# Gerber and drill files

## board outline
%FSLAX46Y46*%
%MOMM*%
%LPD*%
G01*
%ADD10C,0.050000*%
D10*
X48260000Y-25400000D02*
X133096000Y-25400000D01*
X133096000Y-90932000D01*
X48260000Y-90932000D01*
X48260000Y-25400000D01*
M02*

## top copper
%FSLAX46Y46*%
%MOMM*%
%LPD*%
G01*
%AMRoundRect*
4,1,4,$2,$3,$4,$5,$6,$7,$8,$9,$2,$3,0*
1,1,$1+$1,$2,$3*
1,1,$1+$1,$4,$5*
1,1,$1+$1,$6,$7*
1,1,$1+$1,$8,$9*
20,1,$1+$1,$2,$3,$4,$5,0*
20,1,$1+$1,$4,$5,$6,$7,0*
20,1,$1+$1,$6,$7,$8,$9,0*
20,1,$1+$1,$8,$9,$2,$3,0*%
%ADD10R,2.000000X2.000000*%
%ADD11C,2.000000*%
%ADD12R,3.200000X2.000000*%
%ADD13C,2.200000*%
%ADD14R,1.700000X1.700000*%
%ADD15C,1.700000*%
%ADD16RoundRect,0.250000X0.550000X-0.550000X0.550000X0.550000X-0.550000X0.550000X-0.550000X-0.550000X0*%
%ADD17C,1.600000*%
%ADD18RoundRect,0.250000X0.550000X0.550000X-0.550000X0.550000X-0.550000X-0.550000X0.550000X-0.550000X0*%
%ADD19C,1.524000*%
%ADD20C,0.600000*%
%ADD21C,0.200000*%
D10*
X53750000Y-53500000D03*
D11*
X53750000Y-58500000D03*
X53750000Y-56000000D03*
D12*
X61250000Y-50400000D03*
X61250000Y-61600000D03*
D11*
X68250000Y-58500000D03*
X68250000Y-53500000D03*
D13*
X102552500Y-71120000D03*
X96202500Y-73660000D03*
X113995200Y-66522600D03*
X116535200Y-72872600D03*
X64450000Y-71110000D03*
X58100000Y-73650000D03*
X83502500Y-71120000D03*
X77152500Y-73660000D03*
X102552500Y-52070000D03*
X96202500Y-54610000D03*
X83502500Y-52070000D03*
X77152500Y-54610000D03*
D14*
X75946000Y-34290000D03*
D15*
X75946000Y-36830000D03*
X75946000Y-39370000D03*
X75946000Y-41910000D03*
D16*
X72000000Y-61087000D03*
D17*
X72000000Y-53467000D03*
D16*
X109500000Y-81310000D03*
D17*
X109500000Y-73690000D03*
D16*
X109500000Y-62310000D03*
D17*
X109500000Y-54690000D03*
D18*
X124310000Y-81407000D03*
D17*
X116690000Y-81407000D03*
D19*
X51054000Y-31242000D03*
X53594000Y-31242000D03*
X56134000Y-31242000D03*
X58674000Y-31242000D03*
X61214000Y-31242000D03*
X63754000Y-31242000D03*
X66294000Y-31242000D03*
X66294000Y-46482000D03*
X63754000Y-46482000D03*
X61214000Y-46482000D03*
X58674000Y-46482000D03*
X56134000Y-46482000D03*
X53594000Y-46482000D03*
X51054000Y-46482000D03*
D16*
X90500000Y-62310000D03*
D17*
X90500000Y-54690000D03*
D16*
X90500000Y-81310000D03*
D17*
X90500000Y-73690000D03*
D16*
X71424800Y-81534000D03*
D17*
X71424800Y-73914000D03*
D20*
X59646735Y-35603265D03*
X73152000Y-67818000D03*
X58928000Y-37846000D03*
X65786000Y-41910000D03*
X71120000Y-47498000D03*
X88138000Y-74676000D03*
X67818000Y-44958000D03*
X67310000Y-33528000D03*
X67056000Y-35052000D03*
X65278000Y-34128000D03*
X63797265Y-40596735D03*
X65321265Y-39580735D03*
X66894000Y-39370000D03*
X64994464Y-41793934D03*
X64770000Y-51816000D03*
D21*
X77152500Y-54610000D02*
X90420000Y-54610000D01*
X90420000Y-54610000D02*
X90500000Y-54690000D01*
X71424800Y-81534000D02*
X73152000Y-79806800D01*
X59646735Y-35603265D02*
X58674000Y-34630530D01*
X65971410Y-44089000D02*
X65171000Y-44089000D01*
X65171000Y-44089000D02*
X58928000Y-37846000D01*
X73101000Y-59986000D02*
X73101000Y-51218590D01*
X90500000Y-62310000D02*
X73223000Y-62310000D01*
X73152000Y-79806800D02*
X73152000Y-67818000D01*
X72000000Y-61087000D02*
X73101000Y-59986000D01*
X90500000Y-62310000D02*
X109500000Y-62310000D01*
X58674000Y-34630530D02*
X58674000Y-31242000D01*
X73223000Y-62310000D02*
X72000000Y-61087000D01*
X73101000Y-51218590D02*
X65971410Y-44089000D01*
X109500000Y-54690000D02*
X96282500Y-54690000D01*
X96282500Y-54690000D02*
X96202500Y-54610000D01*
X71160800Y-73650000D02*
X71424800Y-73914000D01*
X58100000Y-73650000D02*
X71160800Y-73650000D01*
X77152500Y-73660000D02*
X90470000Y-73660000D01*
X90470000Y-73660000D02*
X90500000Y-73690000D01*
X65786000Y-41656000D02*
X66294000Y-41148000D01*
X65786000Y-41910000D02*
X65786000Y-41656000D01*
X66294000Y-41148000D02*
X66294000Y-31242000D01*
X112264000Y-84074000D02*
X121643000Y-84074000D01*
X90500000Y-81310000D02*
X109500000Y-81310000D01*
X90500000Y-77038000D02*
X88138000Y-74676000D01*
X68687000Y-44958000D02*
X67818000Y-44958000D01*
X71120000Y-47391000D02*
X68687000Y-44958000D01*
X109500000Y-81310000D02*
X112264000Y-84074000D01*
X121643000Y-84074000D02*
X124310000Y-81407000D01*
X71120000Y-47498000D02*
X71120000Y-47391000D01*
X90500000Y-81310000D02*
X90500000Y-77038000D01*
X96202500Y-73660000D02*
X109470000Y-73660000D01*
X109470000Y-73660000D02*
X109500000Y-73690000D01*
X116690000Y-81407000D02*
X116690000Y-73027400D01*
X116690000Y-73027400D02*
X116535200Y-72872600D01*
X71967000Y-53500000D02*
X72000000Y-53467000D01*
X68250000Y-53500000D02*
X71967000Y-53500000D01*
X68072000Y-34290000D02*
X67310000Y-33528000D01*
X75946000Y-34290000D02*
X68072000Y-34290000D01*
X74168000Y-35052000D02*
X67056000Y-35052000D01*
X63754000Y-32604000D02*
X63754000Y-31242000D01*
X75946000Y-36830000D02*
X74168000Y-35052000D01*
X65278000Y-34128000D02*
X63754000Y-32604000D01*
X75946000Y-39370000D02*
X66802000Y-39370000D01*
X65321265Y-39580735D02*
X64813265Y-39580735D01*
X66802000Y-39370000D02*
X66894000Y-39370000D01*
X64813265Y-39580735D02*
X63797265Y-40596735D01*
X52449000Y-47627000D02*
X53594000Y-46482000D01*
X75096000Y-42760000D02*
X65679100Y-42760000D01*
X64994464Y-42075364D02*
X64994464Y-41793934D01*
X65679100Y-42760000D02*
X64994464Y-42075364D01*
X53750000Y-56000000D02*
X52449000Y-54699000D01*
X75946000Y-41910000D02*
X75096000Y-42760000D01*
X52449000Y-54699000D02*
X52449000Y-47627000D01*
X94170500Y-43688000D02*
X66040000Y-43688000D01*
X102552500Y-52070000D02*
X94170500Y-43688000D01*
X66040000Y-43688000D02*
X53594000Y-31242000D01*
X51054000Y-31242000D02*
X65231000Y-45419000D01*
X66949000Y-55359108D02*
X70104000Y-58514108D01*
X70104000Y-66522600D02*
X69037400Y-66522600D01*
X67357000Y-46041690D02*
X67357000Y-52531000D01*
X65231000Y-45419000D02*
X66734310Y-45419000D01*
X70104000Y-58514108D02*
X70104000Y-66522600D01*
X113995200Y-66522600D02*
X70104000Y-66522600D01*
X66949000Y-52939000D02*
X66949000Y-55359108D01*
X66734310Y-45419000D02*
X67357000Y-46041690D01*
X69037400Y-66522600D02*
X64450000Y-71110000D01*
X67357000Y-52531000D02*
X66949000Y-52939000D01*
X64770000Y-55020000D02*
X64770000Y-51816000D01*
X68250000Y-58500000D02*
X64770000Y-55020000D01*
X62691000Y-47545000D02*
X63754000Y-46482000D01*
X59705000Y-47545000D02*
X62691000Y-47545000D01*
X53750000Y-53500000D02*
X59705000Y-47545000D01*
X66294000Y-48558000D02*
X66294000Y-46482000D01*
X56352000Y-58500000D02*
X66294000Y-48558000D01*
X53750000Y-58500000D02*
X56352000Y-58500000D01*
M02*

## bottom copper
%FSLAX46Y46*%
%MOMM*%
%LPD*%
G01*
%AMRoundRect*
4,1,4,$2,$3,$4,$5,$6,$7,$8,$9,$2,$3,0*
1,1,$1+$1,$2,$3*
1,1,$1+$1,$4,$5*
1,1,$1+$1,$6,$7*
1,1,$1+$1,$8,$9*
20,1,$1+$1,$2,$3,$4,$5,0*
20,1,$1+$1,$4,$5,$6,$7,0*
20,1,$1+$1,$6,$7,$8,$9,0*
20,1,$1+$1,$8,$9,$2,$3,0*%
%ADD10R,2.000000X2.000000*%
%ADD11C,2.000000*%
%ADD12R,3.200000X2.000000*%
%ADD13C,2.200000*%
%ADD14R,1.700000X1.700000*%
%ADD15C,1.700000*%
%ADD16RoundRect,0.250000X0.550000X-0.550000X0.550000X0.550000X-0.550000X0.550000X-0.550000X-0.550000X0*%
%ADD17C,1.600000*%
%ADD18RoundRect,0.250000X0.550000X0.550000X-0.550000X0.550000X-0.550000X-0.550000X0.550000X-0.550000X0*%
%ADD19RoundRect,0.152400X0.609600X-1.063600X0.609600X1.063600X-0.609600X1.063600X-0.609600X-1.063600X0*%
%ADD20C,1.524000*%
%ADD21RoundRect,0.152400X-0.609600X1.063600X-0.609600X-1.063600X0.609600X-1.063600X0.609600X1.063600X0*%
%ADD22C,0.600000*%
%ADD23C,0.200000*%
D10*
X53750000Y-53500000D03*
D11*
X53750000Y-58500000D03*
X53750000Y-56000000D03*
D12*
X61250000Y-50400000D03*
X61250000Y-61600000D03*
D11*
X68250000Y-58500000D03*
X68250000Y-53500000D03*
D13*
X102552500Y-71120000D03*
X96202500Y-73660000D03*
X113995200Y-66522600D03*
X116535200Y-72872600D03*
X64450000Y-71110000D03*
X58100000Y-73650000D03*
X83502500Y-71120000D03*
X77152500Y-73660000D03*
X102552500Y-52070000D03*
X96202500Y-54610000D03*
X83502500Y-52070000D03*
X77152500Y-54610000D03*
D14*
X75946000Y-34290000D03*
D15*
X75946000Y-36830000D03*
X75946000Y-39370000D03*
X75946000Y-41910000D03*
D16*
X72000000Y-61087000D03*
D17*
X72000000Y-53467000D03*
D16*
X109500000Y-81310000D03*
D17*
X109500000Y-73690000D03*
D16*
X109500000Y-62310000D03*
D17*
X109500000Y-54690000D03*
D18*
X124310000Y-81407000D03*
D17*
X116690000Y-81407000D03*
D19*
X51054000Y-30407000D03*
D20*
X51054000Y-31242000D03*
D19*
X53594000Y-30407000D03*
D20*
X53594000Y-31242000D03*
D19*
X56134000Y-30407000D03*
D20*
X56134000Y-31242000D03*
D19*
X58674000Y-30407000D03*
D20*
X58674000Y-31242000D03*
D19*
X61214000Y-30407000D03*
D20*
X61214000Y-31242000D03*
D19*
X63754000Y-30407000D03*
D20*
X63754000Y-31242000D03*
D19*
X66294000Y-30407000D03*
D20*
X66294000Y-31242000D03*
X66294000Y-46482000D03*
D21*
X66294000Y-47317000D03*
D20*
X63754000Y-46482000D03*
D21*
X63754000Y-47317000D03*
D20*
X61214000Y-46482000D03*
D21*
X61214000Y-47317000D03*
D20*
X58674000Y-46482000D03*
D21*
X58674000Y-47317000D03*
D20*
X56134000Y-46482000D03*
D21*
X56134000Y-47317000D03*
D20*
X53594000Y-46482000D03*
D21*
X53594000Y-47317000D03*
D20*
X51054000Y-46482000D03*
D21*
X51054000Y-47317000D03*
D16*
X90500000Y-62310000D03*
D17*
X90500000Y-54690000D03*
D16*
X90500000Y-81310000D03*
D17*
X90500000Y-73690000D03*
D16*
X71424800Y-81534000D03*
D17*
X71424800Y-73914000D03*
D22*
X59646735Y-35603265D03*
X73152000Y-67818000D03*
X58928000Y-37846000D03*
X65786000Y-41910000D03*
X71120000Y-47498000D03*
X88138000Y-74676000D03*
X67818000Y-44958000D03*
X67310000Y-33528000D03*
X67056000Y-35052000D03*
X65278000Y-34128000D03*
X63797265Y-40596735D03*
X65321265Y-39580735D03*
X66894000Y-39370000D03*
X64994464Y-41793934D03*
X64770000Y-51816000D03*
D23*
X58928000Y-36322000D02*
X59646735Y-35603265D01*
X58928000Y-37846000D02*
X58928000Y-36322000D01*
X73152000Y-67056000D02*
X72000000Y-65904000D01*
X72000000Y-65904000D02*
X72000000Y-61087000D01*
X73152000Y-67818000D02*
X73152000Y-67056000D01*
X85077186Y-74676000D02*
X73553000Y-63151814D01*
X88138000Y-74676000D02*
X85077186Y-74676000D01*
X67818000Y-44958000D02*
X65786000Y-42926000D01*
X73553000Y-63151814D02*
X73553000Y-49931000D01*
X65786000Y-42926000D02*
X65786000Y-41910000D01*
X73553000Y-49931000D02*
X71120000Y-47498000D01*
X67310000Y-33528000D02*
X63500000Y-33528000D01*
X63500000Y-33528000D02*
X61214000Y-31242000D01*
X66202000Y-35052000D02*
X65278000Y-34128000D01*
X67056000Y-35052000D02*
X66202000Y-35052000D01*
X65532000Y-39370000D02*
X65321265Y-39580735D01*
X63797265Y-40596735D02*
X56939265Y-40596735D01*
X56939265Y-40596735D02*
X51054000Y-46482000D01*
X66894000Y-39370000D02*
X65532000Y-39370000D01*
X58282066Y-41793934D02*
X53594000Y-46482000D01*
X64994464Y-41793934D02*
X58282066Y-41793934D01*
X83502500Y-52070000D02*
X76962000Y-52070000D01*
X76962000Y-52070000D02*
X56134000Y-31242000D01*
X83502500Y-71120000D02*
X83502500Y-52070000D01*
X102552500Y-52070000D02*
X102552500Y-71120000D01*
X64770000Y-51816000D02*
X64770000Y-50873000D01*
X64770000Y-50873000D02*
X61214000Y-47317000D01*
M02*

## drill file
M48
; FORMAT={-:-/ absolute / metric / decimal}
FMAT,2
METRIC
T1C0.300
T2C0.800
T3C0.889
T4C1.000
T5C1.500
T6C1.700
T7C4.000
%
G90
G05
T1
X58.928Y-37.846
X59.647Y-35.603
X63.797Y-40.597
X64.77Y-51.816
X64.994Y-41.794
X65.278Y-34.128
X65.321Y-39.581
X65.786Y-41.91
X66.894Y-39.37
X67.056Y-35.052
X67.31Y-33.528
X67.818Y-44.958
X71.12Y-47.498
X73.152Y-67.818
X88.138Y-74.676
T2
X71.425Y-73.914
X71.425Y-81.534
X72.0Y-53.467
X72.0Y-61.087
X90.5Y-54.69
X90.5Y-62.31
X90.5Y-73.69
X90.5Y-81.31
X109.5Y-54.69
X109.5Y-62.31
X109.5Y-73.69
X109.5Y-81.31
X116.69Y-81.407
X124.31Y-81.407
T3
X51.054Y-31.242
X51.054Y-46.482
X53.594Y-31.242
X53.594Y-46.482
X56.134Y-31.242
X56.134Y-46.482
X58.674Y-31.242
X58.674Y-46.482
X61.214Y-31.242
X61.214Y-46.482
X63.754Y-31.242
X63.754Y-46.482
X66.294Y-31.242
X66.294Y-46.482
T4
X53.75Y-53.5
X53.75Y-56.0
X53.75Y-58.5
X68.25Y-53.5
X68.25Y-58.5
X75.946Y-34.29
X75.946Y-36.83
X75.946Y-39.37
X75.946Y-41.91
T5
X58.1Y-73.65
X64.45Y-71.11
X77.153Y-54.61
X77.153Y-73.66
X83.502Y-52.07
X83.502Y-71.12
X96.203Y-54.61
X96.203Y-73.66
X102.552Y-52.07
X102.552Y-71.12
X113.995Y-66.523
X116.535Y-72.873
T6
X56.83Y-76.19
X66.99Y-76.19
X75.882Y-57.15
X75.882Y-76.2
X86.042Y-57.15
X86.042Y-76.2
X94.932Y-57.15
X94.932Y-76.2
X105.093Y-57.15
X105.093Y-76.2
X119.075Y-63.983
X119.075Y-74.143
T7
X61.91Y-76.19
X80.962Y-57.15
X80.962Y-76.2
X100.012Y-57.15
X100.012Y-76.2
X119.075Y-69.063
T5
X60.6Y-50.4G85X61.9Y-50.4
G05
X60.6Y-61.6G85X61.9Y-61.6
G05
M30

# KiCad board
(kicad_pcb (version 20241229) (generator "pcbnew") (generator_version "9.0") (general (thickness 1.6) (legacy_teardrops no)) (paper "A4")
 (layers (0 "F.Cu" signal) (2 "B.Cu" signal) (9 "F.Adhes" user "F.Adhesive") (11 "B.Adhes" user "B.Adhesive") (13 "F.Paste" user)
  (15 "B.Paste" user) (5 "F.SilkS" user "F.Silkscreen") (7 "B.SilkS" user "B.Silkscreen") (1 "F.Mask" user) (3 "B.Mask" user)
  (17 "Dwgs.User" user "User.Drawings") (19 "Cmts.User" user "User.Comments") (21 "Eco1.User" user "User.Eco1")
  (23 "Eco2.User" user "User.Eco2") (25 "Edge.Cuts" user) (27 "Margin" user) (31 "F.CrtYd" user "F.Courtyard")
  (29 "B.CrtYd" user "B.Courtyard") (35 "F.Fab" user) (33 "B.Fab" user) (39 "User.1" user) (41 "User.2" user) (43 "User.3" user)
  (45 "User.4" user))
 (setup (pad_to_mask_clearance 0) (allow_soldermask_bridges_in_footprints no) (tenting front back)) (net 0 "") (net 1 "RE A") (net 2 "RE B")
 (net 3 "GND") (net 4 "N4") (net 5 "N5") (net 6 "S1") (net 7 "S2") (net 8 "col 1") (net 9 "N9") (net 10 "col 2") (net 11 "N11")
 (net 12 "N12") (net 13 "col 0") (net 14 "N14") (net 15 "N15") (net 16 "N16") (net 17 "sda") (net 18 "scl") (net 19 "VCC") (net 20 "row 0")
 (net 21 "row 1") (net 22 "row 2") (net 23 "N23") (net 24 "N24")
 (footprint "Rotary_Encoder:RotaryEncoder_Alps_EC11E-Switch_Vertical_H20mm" (layer "F.Cu") (at 53.75 53.5)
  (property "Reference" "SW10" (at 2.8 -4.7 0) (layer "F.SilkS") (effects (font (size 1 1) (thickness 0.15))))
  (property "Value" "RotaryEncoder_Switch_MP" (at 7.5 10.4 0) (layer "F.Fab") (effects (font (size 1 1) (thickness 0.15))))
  (pad "A" thru_hole rect (at 0 0) (size 2 2) (drill 1) (layers "*.Cu" "*.Mask") (remove_unused_layers no) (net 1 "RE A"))
  (pad "B" thru_hole circle (at 0 5) (size 2 2) (drill 1) (layers "*.Cu" "*.Mask") (remove_unused_layers no) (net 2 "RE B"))
  (pad "C" thru_hole circle (at 0 2.5) (size 2 2) (drill 1) (layers "*.Cu" "*.Mask") (remove_unused_layers no) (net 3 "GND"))
  (pad "MP" thru_hole rect (at 7.5 -3.1) (size 3.2 2) (drill oval 2.8 1.5) (layers "*.Cu" "*.Mask") (remove_unused_layers no) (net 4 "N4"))
  (pad "MP" thru_hole rect (at 7.5 8.1) (size 3.2 2) (drill oval 2.8 1.5) (layers "*.Cu" "*.Mask") (remove_unused_layers no) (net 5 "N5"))
  (pad "S1" thru_hole circle (at 14.5 5) (size 2 2) (drill 1) (layers "*.Cu" "*.Mask") (remove_unused_layers no) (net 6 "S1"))
  (pad "S2" thru_hole circle (at 14.5 0) (size 2 2) (drill 1) (layers "*.Cu" "*.Mask") (remove_unused_layers no) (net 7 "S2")))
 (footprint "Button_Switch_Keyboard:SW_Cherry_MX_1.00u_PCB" (layer "F.Cu") (at 102.5525 71.12)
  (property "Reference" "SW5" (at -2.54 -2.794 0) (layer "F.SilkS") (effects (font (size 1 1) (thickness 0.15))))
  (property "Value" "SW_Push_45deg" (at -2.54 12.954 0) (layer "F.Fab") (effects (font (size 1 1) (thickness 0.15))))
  (pad "" np_thru_hole circle (at -7.62 5.08) (size 1.7 1.7) (drill 1.7) (layers "*.Cu" "*.Mask"))
  (pad "" np_thru_hole circle (at -2.54 5.08) (size 4 4) (drill 4) (layers "*.Cu" "*.Mask"))
  (pad "" np_thru_hole circle (at 2.54 5.08) (size 1.7 1.7) (drill 1.7) (layers "*.Cu" "*.Mask"))
  (pad "1" thru_hole circle (at 0 0) (size 2.2 2.2) (drill 1.5) (layers "*.Cu" "*.Mask") (remove_unused_layers no) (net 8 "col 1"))
  (pad "2" thru_hole circle (at -6.35 2.54) (size 2.2 2.2) (drill 1.5) (layers "*.Cu" "*.Mask") (remove_unused_layers no) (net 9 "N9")))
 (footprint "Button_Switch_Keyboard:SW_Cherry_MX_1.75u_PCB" (layer "F.Cu") (at 113.9952 66.5226 90)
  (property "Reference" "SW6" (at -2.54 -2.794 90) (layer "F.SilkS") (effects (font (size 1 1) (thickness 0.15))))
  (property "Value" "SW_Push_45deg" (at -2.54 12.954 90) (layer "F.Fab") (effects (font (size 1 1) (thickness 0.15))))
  (pad "" np_thru_hole circle (at -7.62 5.08 90) (size 1.7 1.7) (drill 1.7) (layers "*.Cu" "*.Mask"))
  (pad "" np_thru_hole circle (at -2.54 5.08 90) (size 4 4) (drill 4) (layers "*.Cu" "*.Mask"))
  (pad "" np_thru_hole circle (at 2.54 5.08 90) (size 1.7 1.7) (drill 1.7) (layers "*.Cu" "*.Mask"))
  (pad "1" thru_hole circle (at 0 0 90) (size 2.2 2.2) (drill 1.5) (layers "*.Cu" "*.Mask") (remove_unused_layers no) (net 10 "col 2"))
  (pad "2" thru_hole circle (at -6.35 2.54 90) (size 2.2 2.2) (drill 1.5) (layers "*.Cu" "*.Mask") (remove_unused_layers no) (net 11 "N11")))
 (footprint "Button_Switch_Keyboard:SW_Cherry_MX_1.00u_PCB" (layer "F.Cu") (at 64.45 71.11)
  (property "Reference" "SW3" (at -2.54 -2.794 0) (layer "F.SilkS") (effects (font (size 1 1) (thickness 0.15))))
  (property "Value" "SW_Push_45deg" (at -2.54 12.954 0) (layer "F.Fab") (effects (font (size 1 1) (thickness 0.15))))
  (pad "" np_thru_hole circle (at -7.62 5.08) (size 1.7 1.7) (drill 1.7) (layers "*.Cu" "*.Mask"))
  (pad "" np_thru_hole circle (at -2.54 5.08) (size 4 4) (drill 4) (layers "*.Cu" "*.Mask"))
  (pad "" np_thru_hole circle (at 2.54 5.08) (size 1.7 1.7) (drill 1.7) (layers "*.Cu" "*.Mask"))
  (pad "1" thru_hole circle (at 0 0) (size 2.2 2.2) (drill 1.5) (layers "*.Cu" "*.Mask") (remove_unused_layers no) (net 10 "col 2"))
  (pad "2" thru_hole circle (at -6.35 2.54) (size 2.2 2.2) (drill 1.5) (layers "*.Cu" "*.Mask") (remove_unused_layers no) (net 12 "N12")))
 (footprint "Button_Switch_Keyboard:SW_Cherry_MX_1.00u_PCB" (layer "F.Cu") (at 83.5025 71.12)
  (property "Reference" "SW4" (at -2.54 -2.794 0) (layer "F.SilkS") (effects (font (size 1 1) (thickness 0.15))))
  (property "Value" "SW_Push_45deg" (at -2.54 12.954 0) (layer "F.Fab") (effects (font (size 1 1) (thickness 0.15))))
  (pad "" np_thru_hole circle (at -7.62 5.08) (size 1.7 1.7) (drill 1.7) (layers "*.Cu" "*.Mask"))
  (pad "" np_thru_hole circle (at -2.54 5.08) (size 4 4) (drill 4) (layers "*.Cu" "*.Mask"))
  (pad "" np_thru_hole circle (at 2.54 5.08) (size 1.7 1.7) (drill 1.7) (layers "*.Cu" "*.Mask"))
  (pad "1" thru_hole circle (at 0 0) (size 2.2 2.2) (drill 1.5) (layers "*.Cu" "*.Mask") (remove_unused_layers no) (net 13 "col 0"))
  (pad "2" thru_hole circle (at -6.35 2.54) (size 2.2 2.2) (drill 1.5) (layers "*.Cu" "*.Mask") (remove_unused_layers no) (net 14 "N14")))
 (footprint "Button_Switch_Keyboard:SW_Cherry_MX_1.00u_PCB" (layer "F.Cu") (at 102.5525 52.07)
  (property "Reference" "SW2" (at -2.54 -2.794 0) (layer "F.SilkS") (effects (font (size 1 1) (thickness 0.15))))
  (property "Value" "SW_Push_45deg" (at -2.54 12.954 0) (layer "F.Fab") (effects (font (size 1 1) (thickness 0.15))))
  (pad "" np_thru_hole circle (at -7.62 5.08) (size 1.7 1.7) (drill 1.7) (layers "*.Cu" "*.Mask"))
  (pad "" np_thru_hole circle (at -2.54 5.08) (size 4 4) (drill 4) (layers "*.Cu" "*.Mask"))
  (pad "" np_thru_hole circle (at 2.54 5.08) (size 1.7 1.7) (drill 1.7) (layers "*.Cu" "*.Mask"))
  (pad "1" thru_hole circle (at 0 0) (size 2.2 2.2) (drill 1.5) (layers "*.Cu" "*.Mask") (remove_unused_layers no) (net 8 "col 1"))
  (pad "2" thru_hole circle (at -6.35 2.54) (size 2.2 2.2) (drill 1.5) (layers "*.Cu" "*.Mask") (remove_unused_layers no) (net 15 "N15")))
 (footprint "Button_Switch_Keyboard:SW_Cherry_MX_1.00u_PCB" (layer "F.Cu") (at 83.5025 52.07)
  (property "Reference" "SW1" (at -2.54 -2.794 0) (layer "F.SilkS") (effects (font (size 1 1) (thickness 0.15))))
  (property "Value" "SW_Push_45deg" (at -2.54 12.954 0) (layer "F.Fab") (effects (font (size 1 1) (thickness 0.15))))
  (pad "" np_thru_hole circle (at -7.62 5.08) (size 1.7 1.7) (drill 1.7) (layers "*.Cu" "*.Mask"))
  (pad "" np_thru_hole circle (at -2.54 5.08) (size 4 4) (drill 4) (layers "*.Cu" "*.Mask"))
  (pad "" np_thru_hole circle (at 2.54 5.08) (size 1.7 1.7) (drill 1.7) (layers "*.Cu" "*.Mask"))
  (pad "1" thru_hole circle (at 0 0) (size 2.2 2.2) (drill 1.5) (layers "*.Cu" "*.Mask") (remove_unused_layers no) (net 13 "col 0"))
  (pad "2" thru_hole circle (at -6.35 2.54) (size 2.2 2.2) (drill 1.5) (layers "*.Cu" "*.Mask") (remove_unused_layers no) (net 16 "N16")))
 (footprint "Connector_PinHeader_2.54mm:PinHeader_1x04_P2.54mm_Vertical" (layer "F.Cu") (at 75.946 34.29)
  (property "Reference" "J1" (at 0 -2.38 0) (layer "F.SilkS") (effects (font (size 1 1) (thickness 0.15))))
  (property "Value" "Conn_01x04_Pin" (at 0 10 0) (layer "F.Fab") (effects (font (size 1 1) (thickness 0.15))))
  (pad "1" thru_hole rect (at 0 0) (size 1.7 1.7) (drill 1) (layers "*.Cu" "*.Mask") (remove_unused_layers no) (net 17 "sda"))
  (pad "2" thru_hole circle (at 0 2.54) (size 1.7 1.7) (drill 1) (layers "*.Cu" "*.Mask") (remove_unused_layers no) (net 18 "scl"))
  (pad "3" thru_hole circle (at 0 5.08) (size 1.7 1.7) (drill 1) (layers "*.Cu" "*.Mask") (remove_unused_layers no) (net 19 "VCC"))
  (pad "4" thru_hole circle (at 0 7.62) (size 1.7 1.7) (drill 1) (layers "*.Cu" "*.Mask") (remove_unused_layers no) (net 3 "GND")))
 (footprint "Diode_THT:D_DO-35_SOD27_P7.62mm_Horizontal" (layer "B.Cu") (at 72 61.087 90)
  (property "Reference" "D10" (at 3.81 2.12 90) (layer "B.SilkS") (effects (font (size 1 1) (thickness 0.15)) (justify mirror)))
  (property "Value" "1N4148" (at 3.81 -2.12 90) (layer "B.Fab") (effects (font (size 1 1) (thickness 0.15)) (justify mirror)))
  (pad "1" thru_hole roundrect (at 0 0 90) (size 1.6 1.6) (drill 0.8) (layers "*.Cu" "*.Mask") (remove_unused_layers no)
   (roundrect_rratio 0.15625) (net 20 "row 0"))
  (pad "2" thru_hole circle (at 7.62 0 90) (size 1.6 1.6) (drill 0.8) (layers "*.Cu" "*.Mask") (remove_unused_layers no) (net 7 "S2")))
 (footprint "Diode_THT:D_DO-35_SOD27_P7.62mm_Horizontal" (layer "B.Cu") (at 109.5 81.31 90)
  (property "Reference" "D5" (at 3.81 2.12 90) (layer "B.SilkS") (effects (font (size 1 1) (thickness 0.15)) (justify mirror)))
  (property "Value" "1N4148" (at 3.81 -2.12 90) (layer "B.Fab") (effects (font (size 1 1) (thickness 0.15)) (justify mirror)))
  (pad "1" thru_hole roundrect (at 0 0 90) (size 1.6 1.6) (drill 0.8) (layers "*.Cu" "*.Mask") (remove_unused_layers no)
   (roundrect_rratio 0.15625) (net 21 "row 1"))
  (pad "2" thru_hole circle (at 7.62 0 90) (size 1.6 1.6) (drill 0.8) (layers "*.Cu" "*.Mask") (remove_unused_layers no) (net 9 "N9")))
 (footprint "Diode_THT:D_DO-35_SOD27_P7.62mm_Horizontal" (layer "B.Cu") (at 109.5 62.31 90)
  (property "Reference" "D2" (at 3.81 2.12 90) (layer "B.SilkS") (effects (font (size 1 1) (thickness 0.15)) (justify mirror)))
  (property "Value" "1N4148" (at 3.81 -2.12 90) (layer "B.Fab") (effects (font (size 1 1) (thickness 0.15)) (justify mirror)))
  (pad "1" thru_hole roundrect (at 0 0 90) (size 1.6 1.6) (drill 0.8) (layers "*.Cu" "*.Mask") (remove_unused_layers no)
   (roundrect_rratio 0.15625) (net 20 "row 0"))
  (pad "2" thru_hole circle (at 7.62 0 90) (size 1.6 1.6) (drill 0.8) (layers "*.Cu" "*.Mask") (remove_unused_layers no) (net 15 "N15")))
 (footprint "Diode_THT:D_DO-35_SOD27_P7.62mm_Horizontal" (layer "B.Cu") (at 124.31 81.407 180)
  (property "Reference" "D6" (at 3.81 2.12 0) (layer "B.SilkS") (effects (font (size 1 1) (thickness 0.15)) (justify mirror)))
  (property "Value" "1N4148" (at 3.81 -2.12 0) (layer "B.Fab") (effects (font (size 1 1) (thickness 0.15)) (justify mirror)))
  (pad "1" thru_hole roundrect (at 0 0 180) (size 1.6 1.6) (drill 0.8) (layers "*.Cu" "*.Mask") (remove_unused_layers no)
   (roundrect_rratio 0.15625) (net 21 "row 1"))
  (pad "2" thru_hole circle (at 7.62 0 180) (size 1.6 1.6) (drill 0.8) (layers "*.Cu" "*.Mask") (remove_unused_layers no) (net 11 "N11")))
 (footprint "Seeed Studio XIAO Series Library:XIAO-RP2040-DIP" (layer "B.Cu") (at 58.674 38.862 -90)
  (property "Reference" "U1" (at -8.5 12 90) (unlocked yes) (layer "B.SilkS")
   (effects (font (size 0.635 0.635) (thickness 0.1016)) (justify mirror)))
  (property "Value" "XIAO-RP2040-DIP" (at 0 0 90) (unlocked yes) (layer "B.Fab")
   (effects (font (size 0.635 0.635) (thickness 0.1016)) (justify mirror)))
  (pad "1" smd roundrect (at -8.455 7.62 90) (size 2.432 1.524) (layers "B.Cu" "B.Mask") (roundrect_rratio 0.1) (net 10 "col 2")
   (thermal_bridge_angle 45))
  (pad "1" thru_hole circle (at -7.62 7.62 90) (size 1.524 1.524) (drill 0.889) (layers "*.Cu" "*.Mask") (remove_unused_layers no)
   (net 10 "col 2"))
  (pad "2" smd roundrect (at -8.455 5.08 90) (size 2.432 1.524) (layers "B.Cu" "B.Mask") (roundrect_rratio 0.1) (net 8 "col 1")
   (thermal_bridge_angle 45))
  (pad "2" thru_hole circle (at -7.62 5.08 90) (size 1.524 1.524) (drill 0.889) (layers "*.Cu" "*.Mask") (remove_unused_layers no)
   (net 8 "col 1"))
  (pad "3" smd roundrect (at -8.455 2.54 90) (size 2.432 1.524) (layers "B.Cu" "B.Mask") (roundrect_rratio 0.1) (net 13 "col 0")
   (thermal_bridge_angle 45))
  (pad "3" thru_hole circle (at -7.62 2.54 90) (size 1.524 1.524) (drill 0.889) (layers "*.Cu" "*.Mask") (remove_unused_layers no)
   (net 13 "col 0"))
  (pad "4" smd roundrect (at -8.455 0 90) (size 2.432 1.524) (layers "B.Cu" "B.Mask") (roundrect_rratio 0.1) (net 20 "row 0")
   (thermal_bridge_angle 45))
  (pad "4" thru_hole circle (at -7.62 0 90) (size 1.524 1.524) (drill 0.889) (layers "*.Cu" "*.Mask") (remove_unused_layers no)
   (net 20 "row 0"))
  (pad "5" smd roundrect (at -8.455 -2.54 90) (size 2.432 1.524) (layers "B.Cu" "B.Mask") (roundrect_rratio 0.1) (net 17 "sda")
   (thermal_bridge_angle 45))
  (pad "5" thru_hole circle (at -7.62 -2.54 90) (size 1.524 1.524) (drill 0.889) (layers "*.Cu" "*.Mask") (remove_unused_layers no)
   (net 17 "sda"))
  (pad "6" smd roundrect (at -8.455 -5.08 90) (size 2.432 1.524) (layers "B.Cu" "B.Mask") (roundrect_rratio 0.1) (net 18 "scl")
   (thermal_bridge_angle 45))
  (pad "6" thru_hole circle (at -7.62 -5.08 90) (size 1.524 1.524) (drill 0.889) (layers "*.Cu" "*.Mask") (remove_unused_layers no)
   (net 18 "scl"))
  (pad "7" smd roundrect (at -8.455 -7.62 90) (size 2.432 1.524) (layers "B.Cu" "B.Mask") (roundrect_rratio 0.1) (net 21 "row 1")
   (thermal_bridge_angle 45))
  (pad "7" thru_hole circle (at -7.62 -7.62 90) (size 1.524 1.524) (drill 0.889) (layers "*.Cu" "*.Mask") (remove_unused_layers no)
   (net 21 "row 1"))
  (pad "8" thru_hole circle (at 7.62 -7.62 270) (size 1.524 1.524) (drill 0.889) (layers "*.Cu" "*.Mask") (remove_unused_layers no)
   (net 2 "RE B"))
  (pad "8" smd roundrect (at 8.455 -7.62 270) (size 2.432 1.524) (layers "B.Cu" "B.Mask") (roundrect_rratio 0.1) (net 2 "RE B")
   (thermal_bridge_angle 45))
  (pad "9" thru_hole circle (at 7.62 -5.08 270) (size 1.524 1.524) (drill 0.889) (layers "*.Cu" "*.Mask") (remove_unused_layers no)
   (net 1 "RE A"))
  (pad "9" smd roundrect (at 8.455 -5.08 270) (size 2.432 1.524) (layers "B.Cu" "B.Mask") (roundrect_rratio 0.1) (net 1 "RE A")
   (thermal_bridge_angle 45))
  (pad "10" thru_hole circle (at 7.62 -2.54 270) (size 1.524 1.524) (drill 0.889) (layers "*.Cu" "*.Mask") (remove_unused_layers no)
   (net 6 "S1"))
  (pad "10" smd roundrect (at 8.455 -2.54 270) (size 2.432 1.524) (layers "B.Cu" "B.Mask") (roundrect_rratio 0.1) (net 6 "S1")
   (thermal_bridge_angle 45))
  (pad "11" thru_hole circle (at 7.62 0 270) (size 1.524 1.524) (drill 0.889) (layers "*.Cu" "*.Mask") (remove_unused_layers no)
   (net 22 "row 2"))
  (pad "11" smd roundrect (at 8.455 0 270) (size 2.432 1.524) (layers "B.Cu" "B.Mask") (roundrect_rratio 0.1) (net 22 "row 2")
   (thermal_bridge_angle 45))
  (pad "12" thru_hole circle (at 7.62 2.54 270) (size 1.524 1.524) (drill 0.889) (layers "*.Cu" "*.Mask") (remove_unused_layers no)
   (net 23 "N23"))
  (pad "12" smd roundrect (at 8.455 2.54 270) (size 2.432 1.524) (layers "B.Cu" "B.Mask") (roundrect_rratio 0.1) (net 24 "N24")
   (thermal_bridge_angle 45))
  (pad "13" thru_hole circle (at 7.62 5.08 270) (size 1.524 1.524) (drill 0.889) (layers "*.Cu" "*.Mask") (remove_unused_layers no)
   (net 3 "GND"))
  (pad "13" smd roundrect (at 8.455 5.08 270) (size 2.432 1.524) (layers "B.Cu" "B.Mask") (roundrect_rratio 0.1) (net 3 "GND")
   (thermal_bridge_angle 45))
  (pad "14" thru_hole circle (at 7.62 7.62 270) (size 1.524 1.524) (drill 0.889) (layers "*.Cu" "*.Mask") (remove_unused_layers no)
   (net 19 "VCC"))
  (pad "14" smd roundrect (at 8.455 7.62 270) (size 2.432 1.524) (layers "B.Cu" "B.Mask") (roundrect_rratio 0.1) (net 19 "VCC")
   (thermal_bridge_angle 45)))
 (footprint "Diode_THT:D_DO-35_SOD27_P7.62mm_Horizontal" (layer "B.Cu") (at 90.5 62.31 90)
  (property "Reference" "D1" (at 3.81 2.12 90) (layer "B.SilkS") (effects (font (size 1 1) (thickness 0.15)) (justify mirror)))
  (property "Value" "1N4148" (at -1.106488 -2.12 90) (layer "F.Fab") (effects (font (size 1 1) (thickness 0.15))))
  (pad "1" thru_hole roundrect (at 0 0 90) (size 1.6 1.6) (drill 0.8) (layers "*.Cu" "*.Mask") (remove_unused_layers no)
   (roundrect_rratio 0.15625) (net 20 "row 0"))
  (pad "2" thru_hole circle (at 7.62 0 90) (size 1.6 1.6) (drill 0.8) (layers "*.Cu" "*.Mask") (remove_unused_layers no) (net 16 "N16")))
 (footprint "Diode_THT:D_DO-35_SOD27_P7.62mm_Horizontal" (layer "B.Cu") (at 90.5 81.31 90)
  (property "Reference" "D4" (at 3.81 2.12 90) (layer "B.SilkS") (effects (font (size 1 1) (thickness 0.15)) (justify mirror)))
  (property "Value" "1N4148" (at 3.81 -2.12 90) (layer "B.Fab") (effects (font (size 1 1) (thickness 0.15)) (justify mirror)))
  (pad "1" thru_hole roundrect (at 0 0 90) (size 1.6 1.6) (drill 0.8) (layers "*.Cu" "*.Mask") (remove_unused_layers no)
   (roundrect_rratio 0.15625) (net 21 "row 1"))
  (pad "2" thru_hole circle (at 7.62 0 90) (size 1.6 1.6) (drill 0.8) (layers "*.Cu" "*.Mask") (remove_unused_layers no) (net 14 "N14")))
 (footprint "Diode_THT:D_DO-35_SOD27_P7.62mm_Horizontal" (layer "B.Cu") (at 71.4248 81.534 90)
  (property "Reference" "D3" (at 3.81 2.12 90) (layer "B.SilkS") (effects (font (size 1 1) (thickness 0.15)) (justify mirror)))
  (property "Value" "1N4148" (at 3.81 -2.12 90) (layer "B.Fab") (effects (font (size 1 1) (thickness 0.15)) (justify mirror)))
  (pad "1" thru_hole roundrect (at 0 0 90) (size 1.6 1.6) (drill 0.8) (layers "*.Cu" "*.Mask") (remove_unused_layers no)
   (roundrect_rratio 0.15625) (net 20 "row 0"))
  (pad "2" thru_hole circle (at 7.62 0 90) (size 1.6 1.6) (drill 0.8) (layers "*.Cu" "*.Mask") (remove_unused_layers no) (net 12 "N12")))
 (gr_rect (start 48.26 25.4) (end 133.096 90.932) (stroke (width 0.05) (type default)) (fill no) (layer "Edge.Cuts"))
 (segment (start 77.1525 54.61) (end 90.42 54.61) (width 0.2) (layer "F.Cu") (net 16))
 (segment (start 90.42 54.61) (end 90.5 54.69) (width 0.2) (layer "F.Cu") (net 16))
 (segment (start 71.4248 81.534) (end 73.152 79.8068) (width 0.2) (layer "F.Cu") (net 20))
 (segment (start 59.646735 35.603265) (end 58.674 34.63053) (width 0.2) (layer "F.Cu") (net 20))
 (segment (start 65.97141 44.089) (end 65.171 44.089) (width 0.2) (layer "F.Cu") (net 20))
 (segment (start 65.171 44.089) (end 58.928 37.846) (width 0.2) (layer "F.Cu") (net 20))
 (segment (start 73.101 59.986) (end 73.101 51.21859) (width 0.2) (layer "F.Cu") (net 20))
 (segment (start 90.5 62.31) (end 73.223 62.31) (width 0.2) (layer "F.Cu") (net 20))
 (segment (start 73.152 79.8068) (end 73.152 67.818) (width 0.2) (layer "F.Cu") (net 20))
 (segment (start 72 61.087) (end 73.101 59.986) (width 0.2) (layer "F.Cu") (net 20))
 (segment (start 90.5 62.31) (end 109.5 62.31) (width 0.2) (layer "F.Cu") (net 20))
 (segment (start 58.674 34.63053) (end 58.674 31.242) (width 0.2) (layer "F.Cu") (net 20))
 (segment (start 73.223 62.31) (end 72 61.087) (width 0.2) (layer "F.Cu") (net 20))
 (segment (start 73.101 51.21859) (end 65.97141 44.089) (width 0.2) (layer "F.Cu") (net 20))
 (via (at 59.646735 35.603265) (size 0.6) (drill 0.3) (layers "F.Cu" "B.Cu") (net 20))
 (via (at 73.152 67.818) (size 0.6) (drill 0.3) (layers "F.Cu" "B.Cu") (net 20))
 (via (at 58.928 37.846) (size 0.6) (drill 0.3) (layers "F.Cu" "B.Cu") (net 20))
 (segment (start 58.928 36.322) (end 59.646735 35.603265) (width 0.2) (layer "B.Cu") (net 20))
 (segment (start 58.928 37.846) (end 58.928 36.322) (width 0.2) (layer "B.Cu") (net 20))
 (segment (start 73.152 67.056) (end 72 65.904) (width 0.2) (layer "B.Cu") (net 20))
 (segment (start 72 65.904) (end 72 61.087) (width 0.2) (layer "B.Cu") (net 20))
 (segment (start 73.152 67.818) (end 73.152 67.056) (width 0.2) (layer "B.Cu") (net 20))
 (segment (start 109.5 54.69) (end 96.2825 54.69) (width 0.2) (layer "F.Cu") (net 15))
 (segment (start 96.2825 54.69) (end 96.2025 54.61) (width 0.2) (layer "F.Cu") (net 15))
 (segment (start 71.1608 73.65) (end 71.4248 73.914) (width 0.2) (layer "F.Cu") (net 12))
 (segment (start 58.1 73.65) (end 71.1608 73.65) (width 0.2) (layer "F.Cu") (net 12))
 (segment (start 77.1525 73.66) (end 90.47 73.66) (width 0.2) (layer "F.Cu") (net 14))
 (segment (start 90.47 73.66) (end 90.5 73.69) (width 0.2) (layer "F.Cu") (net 14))
 (segment (start 65.786 41.656) (end 66.294 41.148) (width 0.2) (layer "F.Cu") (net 21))
 (segment (start 65.786 41.91) (end 65.786 41.656) (width 0.2) (layer "F.Cu") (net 21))
 (segment (start 66.294 41.148) (end 66.294 31.242) (width 0.2) (layer "F.Cu") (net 21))
 (segment (start 112.264 84.074) (end 121.643 84.074) (width 0.2) (layer "F.Cu") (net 21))
 (segment (start 90.5 81.31) (end 109.5 81.31) (width 0.2) (layer "F.Cu") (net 21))
 (segment (start 90.5 77.038) (end 88.138 74.676) (width 0.2) (layer "F.Cu") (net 21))
 (segment (start 68.687 44.958) (end 67.818 44.958) (width 0.2) (layer "F.Cu") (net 21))
 (segment (start 71.12 47.391) (end 68.687 44.958) (width 0.2) (layer "F.Cu") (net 21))
 (segment (start 109.5 81.31) (end 112.264 84.074) (width 0.2) (layer "F.Cu") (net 21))
 (segment (start 121.643 84.074) (end 124.31 81.407) (width 0.2) (layer "F.Cu") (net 21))
 (segment (start 71.12 47.498) (end 71.12 47.391) (width 0.2) (layer "F.Cu") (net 21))
 (segment (start 90.5 81.31) (end 90.5 77.038) (width 0.2) (layer "F.Cu") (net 21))
 (via (at 65.786 41.91) (size 0.6) (drill 0.3) (layers "F.Cu" "B.Cu") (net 21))
 (via (at 71.12 47.498) (size 0.6) (drill 0.3) (layers "F.Cu" "B.Cu") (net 21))
 (via (at 88.138 74.676) (size 0.6) (drill 0.3) (layers "F.Cu" "B.Cu") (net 21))
 (via (at 67.818 44.958) (size 0.6) (drill 0.3) (layers "F.Cu" "B.Cu") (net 21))
 (segment (start 85.077186 74.676) (end 73.553 63.151814) (width 0.2) (layer "B.Cu") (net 21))
 (segment (start 88.138 74.676) (end 85.077186 74.676) (width 0.2) (layer "B.Cu") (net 21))
 (segment (start 67.818 44.958) (end 65.786 42.926) (width 0.2) (layer "B.Cu") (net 21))
 (segment (start 73.553 63.151814) (end 73.553 49.931) (width 0.2) (layer "B.Cu") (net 21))
 (segment (start 65.786 42.926) (end 65.786 41.91) (width 0.2) (layer "B.Cu") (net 21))
 (segment (start 73.553 49.931) (end 71.12 47.498) (width 0.2) (layer "B.Cu") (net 21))
 (segment (start 96.2025 73.66) (end 109.47 73.66) (width 0.2) (layer "F.Cu") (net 9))
 (segment (start 109.47 73.66) (end 109.5 73.69) (width 0.2) (layer "F.Cu") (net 9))
 (segment (start 116.69 81.407) (end 116.69 73.0274) (width 0.2) (layer "F.Cu") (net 11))
 (segment (start 116.69 73.0274) (end 116.5352 72.8726) (width 0.2) (layer "F.Cu") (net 11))
 (segment (start 71.967 53.5) (end 72 53.467) (width 0.2) (layer "F.Cu") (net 7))
 (segment (start 68.25 53.5) (end 71.967 53.5) (width 0.2) (layer "F.Cu") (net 7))
 (segment (start 68.072 34.29) (end 67.31 33.528) (width 0.2) (layer "F.Cu") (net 17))
 (segment (start 75.946 34.29) (end 68.072 34.29) (width 0.2) (layer "F.Cu") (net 17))
 (via (at 67.31 33.528) (size 0.6) (drill 0.3) (layers "F.Cu" "B.Cu") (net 17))
 (segment (start 67.31 33.528) (end 63.5 33.528) (width 0.2) (layer "B.Cu") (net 17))
 (segment (start 63.5 33.528) (end 61.214 31.242) (width 0.2) (layer "B.Cu") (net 17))
 (segment (start 74.168 35.052) (end 67.056 35.052) (width 0.2) (layer "F.Cu") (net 18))
 (segment (start 63.754 32.604) (end 63.754 31.242) (width 0.2) (layer "F.Cu") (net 18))
 (segment (start 75.946 36.83) (end 74.168 35.052) (width 0.2) (layer "F.Cu") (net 18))
 (segment (start 65.278 34.128) (end 63.754 32.604) (width 0.2) (layer "F.Cu") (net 18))
 (via (at 67.056 35.052) (size 0.6) (drill 0.3) (layers "F.Cu" "B.Cu") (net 18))
 (via (at 65.278 34.128) (size 0.6) (drill 0.3) (layers "F.Cu" "B.Cu") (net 18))
 (segment (start 66.202 35.052) (end 65.278 34.128) (width 0.2) (layer "B.Cu") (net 18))
 (segment (start 67.056 35.052) (end 66.202 35.052) (width 0.2) (layer "B.Cu") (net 18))
 (segment (start 75.946 39.37) (end 66.802 39.37) (width 0.2) (layer "F.Cu") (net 19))
 (segment (start 65.321265 39.580735) (end 64.813265 39.580735) (width 0.2) (layer "F.Cu") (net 19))
 (segment (start 66.802 39.37) (end 66.894 39.37) (width 0.2) (layer "F.Cu") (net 19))
 (segment (start 64.813265 39.580735) (end 63.797265 40.596735) (width 0.2) (layer "F.Cu") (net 19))
 (via (at 63.797265 40.596735) (size 0.6) (drill 0.3) (layers "F.Cu" "B.Cu") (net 19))
 (via (at 65.321265 39.580735) (size 0.6) (drill 0.3) (layers "F.Cu" "B.Cu") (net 19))
 (via (at 66.894 39.37) (size 0.6) (drill 0.3) (layers "F.Cu" "B.Cu") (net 19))
 (segment (start 65.532 39.37) (end 65.321265 39.580735) (width 0.2) (layer "B.Cu") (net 19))
 (segment (start 63.797265 40.596735) (end 56.939265 40.596735) (width 0.2) (layer "B.Cu") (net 19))
 (segment (start 56.939265 40.596735) (end 51.054 46.482) (width 0.2) (layer "B.Cu") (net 19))
 (segment (start 66.894 39.37) (end 65.532 39.37) (width 0.2) (layer "B.Cu") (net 19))
 (segment (start 52.449 47.627) (end 53.594 46.482) (width 0.2) (layer "F.Cu") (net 3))
 (segment (start 75.096 42.76) (end 65.6791 42.76) (width 0.2) (layer "F.Cu") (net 3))
 (segment (start 64.994464 42.075364) (end 64.994464 41.793934) (width 0.2) (layer "F.Cu") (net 3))
 (segment (start 65.6791 42.76) (end 64.994464 42.075364) (width 0.2) (layer "F.Cu") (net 3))
 (segment (start 53.75 56) (end 52.449 54.699) (width 0.2) (layer "F.Cu") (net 3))
 (segment (start 75.946 41.91) (end 75.096 42.76) (width 0.2) (layer "F.Cu") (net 3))
 (segment (start 52.449 54.699) (end 52.449 47.627) (width 0.2) (layer "F.Cu") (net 3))
 (via (at 64.994464 41.793934) (size 0.6) (drill 0.3) (layers "F.Cu" "B.Cu") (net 3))
 (segment (start 58.282066 41.793934) (end 53.594 46.482) (width 0.2) (layer "B.Cu") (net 3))
 (segment (start 64.994464 41.793934) (end 58.282066 41.793934) (width 0.2) (layer "B.Cu") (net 3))
 (segment (start 83.5025 52.07) (end 76.962 52.07) (width 0.2) (layer "B.Cu") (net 13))
 (segment (start 76.962 52.07) (end 56.134 31.242) (width 0.2) (layer "B.Cu") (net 13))
 (segment (start 83.5025 71.12) (end 83.5025 52.07) (width 0.2) (layer "B.Cu") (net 13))
 (segment (start 94.1705 43.688) (end 66.04 43.688) (width 0.2) (layer "F.Cu") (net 8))
 (segment (start 102.5525 52.07) (end 94.1705 43.688) (width 0.2) (layer "F.Cu") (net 8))
 (segment (start 66.04 43.688) (end 53.594 31.242) (width 0.2) (layer "F.Cu") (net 8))
 (segment (start 102.5525 52.07) (end 102.5525 71.12) (width 0.2) (layer "B.Cu") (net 8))
 (segment (start 51.054 31.242) (end 65.231 45.419) (width 0.2) (layer "F.Cu") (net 10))
 (segment (start 66.949 55.359108) (end 70.104 58.514108) (width 0.2) (layer "F.Cu") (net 10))
 (segment (start 70.104 66.5226) (end 69.0374 66.5226) (width 0.2) (layer "F.Cu") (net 10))
 (segment (start 67.357 46.04169) (end 67.357 52.531) (width 0.2) (layer "F.Cu") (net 10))
 (segment (start 65.231 45.419) (end 66.73431 45.419) (width 0.2) (layer "F.Cu") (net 10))
 (segment (start 70.104 58.514108) (end 70.104 66.5226) (width 0.2) (layer "F.Cu") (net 10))
 (segment (start 113.9952 66.5226) (end 70.104 66.5226) (width 0.2) (layer "F.Cu") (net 10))
 (segment (start 66.949 52.939) (end 66.949 55.359108) (width 0.2) (layer "F.Cu") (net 10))
 (segment (start 66.73431 45.419) (end 67.357 46.04169) (width 0.2) (layer "F.Cu") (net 10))
 (segment (start 69.0374 66.5226) (end 64.45 71.11) (width 0.2) (layer "F.Cu") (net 10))
 (segment (start 67.357 52.531) (end 66.949 52.939) (width 0.2) (layer "F.Cu") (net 10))
 (segment (start 64.77 55.02) (end 64.77 51.816) (width 0.2) (layer "F.Cu") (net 6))
 (segment (start 68.25 58.5) (end 64.77 55.02) (width 0.2) (layer "F.Cu") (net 6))
 (via (at 64.77 51.816) (size 0.6) (drill 0.3) (layers "F.Cu" "B.Cu") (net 6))
 (segment (start 64.77 51.816) (end 64.77 50.873) (width 0.2) (layer "B.Cu") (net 6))
 (segment (start 64.77 50.873) (end 61.214 47.317) (width 0.2) (layer "B.Cu") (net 6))
 (segment (start 62.691 47.545) (end 63.754 46.482) (width 0.2) (layer "F.Cu") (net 1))
 (segment (start 59.705 47.545) (end 62.691 47.545) (width 0.2) (layer "F.Cu") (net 1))
 (segment (start 53.75 53.5) (end 59.705 47.545) (width 0.2) (layer "F.Cu") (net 1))
 (segment (start 66.294 48.558) (end 66.294 46.482) (width 0.2) (layer "F.Cu") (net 2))
 (segment (start 56.352 58.5) (end 66.294 48.558) (width 0.2) (layer "F.Cu") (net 2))
 (segment (start 53.75 58.5) (end 56.352 58.5) (width 0.2) (layer "F.Cu") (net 2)))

